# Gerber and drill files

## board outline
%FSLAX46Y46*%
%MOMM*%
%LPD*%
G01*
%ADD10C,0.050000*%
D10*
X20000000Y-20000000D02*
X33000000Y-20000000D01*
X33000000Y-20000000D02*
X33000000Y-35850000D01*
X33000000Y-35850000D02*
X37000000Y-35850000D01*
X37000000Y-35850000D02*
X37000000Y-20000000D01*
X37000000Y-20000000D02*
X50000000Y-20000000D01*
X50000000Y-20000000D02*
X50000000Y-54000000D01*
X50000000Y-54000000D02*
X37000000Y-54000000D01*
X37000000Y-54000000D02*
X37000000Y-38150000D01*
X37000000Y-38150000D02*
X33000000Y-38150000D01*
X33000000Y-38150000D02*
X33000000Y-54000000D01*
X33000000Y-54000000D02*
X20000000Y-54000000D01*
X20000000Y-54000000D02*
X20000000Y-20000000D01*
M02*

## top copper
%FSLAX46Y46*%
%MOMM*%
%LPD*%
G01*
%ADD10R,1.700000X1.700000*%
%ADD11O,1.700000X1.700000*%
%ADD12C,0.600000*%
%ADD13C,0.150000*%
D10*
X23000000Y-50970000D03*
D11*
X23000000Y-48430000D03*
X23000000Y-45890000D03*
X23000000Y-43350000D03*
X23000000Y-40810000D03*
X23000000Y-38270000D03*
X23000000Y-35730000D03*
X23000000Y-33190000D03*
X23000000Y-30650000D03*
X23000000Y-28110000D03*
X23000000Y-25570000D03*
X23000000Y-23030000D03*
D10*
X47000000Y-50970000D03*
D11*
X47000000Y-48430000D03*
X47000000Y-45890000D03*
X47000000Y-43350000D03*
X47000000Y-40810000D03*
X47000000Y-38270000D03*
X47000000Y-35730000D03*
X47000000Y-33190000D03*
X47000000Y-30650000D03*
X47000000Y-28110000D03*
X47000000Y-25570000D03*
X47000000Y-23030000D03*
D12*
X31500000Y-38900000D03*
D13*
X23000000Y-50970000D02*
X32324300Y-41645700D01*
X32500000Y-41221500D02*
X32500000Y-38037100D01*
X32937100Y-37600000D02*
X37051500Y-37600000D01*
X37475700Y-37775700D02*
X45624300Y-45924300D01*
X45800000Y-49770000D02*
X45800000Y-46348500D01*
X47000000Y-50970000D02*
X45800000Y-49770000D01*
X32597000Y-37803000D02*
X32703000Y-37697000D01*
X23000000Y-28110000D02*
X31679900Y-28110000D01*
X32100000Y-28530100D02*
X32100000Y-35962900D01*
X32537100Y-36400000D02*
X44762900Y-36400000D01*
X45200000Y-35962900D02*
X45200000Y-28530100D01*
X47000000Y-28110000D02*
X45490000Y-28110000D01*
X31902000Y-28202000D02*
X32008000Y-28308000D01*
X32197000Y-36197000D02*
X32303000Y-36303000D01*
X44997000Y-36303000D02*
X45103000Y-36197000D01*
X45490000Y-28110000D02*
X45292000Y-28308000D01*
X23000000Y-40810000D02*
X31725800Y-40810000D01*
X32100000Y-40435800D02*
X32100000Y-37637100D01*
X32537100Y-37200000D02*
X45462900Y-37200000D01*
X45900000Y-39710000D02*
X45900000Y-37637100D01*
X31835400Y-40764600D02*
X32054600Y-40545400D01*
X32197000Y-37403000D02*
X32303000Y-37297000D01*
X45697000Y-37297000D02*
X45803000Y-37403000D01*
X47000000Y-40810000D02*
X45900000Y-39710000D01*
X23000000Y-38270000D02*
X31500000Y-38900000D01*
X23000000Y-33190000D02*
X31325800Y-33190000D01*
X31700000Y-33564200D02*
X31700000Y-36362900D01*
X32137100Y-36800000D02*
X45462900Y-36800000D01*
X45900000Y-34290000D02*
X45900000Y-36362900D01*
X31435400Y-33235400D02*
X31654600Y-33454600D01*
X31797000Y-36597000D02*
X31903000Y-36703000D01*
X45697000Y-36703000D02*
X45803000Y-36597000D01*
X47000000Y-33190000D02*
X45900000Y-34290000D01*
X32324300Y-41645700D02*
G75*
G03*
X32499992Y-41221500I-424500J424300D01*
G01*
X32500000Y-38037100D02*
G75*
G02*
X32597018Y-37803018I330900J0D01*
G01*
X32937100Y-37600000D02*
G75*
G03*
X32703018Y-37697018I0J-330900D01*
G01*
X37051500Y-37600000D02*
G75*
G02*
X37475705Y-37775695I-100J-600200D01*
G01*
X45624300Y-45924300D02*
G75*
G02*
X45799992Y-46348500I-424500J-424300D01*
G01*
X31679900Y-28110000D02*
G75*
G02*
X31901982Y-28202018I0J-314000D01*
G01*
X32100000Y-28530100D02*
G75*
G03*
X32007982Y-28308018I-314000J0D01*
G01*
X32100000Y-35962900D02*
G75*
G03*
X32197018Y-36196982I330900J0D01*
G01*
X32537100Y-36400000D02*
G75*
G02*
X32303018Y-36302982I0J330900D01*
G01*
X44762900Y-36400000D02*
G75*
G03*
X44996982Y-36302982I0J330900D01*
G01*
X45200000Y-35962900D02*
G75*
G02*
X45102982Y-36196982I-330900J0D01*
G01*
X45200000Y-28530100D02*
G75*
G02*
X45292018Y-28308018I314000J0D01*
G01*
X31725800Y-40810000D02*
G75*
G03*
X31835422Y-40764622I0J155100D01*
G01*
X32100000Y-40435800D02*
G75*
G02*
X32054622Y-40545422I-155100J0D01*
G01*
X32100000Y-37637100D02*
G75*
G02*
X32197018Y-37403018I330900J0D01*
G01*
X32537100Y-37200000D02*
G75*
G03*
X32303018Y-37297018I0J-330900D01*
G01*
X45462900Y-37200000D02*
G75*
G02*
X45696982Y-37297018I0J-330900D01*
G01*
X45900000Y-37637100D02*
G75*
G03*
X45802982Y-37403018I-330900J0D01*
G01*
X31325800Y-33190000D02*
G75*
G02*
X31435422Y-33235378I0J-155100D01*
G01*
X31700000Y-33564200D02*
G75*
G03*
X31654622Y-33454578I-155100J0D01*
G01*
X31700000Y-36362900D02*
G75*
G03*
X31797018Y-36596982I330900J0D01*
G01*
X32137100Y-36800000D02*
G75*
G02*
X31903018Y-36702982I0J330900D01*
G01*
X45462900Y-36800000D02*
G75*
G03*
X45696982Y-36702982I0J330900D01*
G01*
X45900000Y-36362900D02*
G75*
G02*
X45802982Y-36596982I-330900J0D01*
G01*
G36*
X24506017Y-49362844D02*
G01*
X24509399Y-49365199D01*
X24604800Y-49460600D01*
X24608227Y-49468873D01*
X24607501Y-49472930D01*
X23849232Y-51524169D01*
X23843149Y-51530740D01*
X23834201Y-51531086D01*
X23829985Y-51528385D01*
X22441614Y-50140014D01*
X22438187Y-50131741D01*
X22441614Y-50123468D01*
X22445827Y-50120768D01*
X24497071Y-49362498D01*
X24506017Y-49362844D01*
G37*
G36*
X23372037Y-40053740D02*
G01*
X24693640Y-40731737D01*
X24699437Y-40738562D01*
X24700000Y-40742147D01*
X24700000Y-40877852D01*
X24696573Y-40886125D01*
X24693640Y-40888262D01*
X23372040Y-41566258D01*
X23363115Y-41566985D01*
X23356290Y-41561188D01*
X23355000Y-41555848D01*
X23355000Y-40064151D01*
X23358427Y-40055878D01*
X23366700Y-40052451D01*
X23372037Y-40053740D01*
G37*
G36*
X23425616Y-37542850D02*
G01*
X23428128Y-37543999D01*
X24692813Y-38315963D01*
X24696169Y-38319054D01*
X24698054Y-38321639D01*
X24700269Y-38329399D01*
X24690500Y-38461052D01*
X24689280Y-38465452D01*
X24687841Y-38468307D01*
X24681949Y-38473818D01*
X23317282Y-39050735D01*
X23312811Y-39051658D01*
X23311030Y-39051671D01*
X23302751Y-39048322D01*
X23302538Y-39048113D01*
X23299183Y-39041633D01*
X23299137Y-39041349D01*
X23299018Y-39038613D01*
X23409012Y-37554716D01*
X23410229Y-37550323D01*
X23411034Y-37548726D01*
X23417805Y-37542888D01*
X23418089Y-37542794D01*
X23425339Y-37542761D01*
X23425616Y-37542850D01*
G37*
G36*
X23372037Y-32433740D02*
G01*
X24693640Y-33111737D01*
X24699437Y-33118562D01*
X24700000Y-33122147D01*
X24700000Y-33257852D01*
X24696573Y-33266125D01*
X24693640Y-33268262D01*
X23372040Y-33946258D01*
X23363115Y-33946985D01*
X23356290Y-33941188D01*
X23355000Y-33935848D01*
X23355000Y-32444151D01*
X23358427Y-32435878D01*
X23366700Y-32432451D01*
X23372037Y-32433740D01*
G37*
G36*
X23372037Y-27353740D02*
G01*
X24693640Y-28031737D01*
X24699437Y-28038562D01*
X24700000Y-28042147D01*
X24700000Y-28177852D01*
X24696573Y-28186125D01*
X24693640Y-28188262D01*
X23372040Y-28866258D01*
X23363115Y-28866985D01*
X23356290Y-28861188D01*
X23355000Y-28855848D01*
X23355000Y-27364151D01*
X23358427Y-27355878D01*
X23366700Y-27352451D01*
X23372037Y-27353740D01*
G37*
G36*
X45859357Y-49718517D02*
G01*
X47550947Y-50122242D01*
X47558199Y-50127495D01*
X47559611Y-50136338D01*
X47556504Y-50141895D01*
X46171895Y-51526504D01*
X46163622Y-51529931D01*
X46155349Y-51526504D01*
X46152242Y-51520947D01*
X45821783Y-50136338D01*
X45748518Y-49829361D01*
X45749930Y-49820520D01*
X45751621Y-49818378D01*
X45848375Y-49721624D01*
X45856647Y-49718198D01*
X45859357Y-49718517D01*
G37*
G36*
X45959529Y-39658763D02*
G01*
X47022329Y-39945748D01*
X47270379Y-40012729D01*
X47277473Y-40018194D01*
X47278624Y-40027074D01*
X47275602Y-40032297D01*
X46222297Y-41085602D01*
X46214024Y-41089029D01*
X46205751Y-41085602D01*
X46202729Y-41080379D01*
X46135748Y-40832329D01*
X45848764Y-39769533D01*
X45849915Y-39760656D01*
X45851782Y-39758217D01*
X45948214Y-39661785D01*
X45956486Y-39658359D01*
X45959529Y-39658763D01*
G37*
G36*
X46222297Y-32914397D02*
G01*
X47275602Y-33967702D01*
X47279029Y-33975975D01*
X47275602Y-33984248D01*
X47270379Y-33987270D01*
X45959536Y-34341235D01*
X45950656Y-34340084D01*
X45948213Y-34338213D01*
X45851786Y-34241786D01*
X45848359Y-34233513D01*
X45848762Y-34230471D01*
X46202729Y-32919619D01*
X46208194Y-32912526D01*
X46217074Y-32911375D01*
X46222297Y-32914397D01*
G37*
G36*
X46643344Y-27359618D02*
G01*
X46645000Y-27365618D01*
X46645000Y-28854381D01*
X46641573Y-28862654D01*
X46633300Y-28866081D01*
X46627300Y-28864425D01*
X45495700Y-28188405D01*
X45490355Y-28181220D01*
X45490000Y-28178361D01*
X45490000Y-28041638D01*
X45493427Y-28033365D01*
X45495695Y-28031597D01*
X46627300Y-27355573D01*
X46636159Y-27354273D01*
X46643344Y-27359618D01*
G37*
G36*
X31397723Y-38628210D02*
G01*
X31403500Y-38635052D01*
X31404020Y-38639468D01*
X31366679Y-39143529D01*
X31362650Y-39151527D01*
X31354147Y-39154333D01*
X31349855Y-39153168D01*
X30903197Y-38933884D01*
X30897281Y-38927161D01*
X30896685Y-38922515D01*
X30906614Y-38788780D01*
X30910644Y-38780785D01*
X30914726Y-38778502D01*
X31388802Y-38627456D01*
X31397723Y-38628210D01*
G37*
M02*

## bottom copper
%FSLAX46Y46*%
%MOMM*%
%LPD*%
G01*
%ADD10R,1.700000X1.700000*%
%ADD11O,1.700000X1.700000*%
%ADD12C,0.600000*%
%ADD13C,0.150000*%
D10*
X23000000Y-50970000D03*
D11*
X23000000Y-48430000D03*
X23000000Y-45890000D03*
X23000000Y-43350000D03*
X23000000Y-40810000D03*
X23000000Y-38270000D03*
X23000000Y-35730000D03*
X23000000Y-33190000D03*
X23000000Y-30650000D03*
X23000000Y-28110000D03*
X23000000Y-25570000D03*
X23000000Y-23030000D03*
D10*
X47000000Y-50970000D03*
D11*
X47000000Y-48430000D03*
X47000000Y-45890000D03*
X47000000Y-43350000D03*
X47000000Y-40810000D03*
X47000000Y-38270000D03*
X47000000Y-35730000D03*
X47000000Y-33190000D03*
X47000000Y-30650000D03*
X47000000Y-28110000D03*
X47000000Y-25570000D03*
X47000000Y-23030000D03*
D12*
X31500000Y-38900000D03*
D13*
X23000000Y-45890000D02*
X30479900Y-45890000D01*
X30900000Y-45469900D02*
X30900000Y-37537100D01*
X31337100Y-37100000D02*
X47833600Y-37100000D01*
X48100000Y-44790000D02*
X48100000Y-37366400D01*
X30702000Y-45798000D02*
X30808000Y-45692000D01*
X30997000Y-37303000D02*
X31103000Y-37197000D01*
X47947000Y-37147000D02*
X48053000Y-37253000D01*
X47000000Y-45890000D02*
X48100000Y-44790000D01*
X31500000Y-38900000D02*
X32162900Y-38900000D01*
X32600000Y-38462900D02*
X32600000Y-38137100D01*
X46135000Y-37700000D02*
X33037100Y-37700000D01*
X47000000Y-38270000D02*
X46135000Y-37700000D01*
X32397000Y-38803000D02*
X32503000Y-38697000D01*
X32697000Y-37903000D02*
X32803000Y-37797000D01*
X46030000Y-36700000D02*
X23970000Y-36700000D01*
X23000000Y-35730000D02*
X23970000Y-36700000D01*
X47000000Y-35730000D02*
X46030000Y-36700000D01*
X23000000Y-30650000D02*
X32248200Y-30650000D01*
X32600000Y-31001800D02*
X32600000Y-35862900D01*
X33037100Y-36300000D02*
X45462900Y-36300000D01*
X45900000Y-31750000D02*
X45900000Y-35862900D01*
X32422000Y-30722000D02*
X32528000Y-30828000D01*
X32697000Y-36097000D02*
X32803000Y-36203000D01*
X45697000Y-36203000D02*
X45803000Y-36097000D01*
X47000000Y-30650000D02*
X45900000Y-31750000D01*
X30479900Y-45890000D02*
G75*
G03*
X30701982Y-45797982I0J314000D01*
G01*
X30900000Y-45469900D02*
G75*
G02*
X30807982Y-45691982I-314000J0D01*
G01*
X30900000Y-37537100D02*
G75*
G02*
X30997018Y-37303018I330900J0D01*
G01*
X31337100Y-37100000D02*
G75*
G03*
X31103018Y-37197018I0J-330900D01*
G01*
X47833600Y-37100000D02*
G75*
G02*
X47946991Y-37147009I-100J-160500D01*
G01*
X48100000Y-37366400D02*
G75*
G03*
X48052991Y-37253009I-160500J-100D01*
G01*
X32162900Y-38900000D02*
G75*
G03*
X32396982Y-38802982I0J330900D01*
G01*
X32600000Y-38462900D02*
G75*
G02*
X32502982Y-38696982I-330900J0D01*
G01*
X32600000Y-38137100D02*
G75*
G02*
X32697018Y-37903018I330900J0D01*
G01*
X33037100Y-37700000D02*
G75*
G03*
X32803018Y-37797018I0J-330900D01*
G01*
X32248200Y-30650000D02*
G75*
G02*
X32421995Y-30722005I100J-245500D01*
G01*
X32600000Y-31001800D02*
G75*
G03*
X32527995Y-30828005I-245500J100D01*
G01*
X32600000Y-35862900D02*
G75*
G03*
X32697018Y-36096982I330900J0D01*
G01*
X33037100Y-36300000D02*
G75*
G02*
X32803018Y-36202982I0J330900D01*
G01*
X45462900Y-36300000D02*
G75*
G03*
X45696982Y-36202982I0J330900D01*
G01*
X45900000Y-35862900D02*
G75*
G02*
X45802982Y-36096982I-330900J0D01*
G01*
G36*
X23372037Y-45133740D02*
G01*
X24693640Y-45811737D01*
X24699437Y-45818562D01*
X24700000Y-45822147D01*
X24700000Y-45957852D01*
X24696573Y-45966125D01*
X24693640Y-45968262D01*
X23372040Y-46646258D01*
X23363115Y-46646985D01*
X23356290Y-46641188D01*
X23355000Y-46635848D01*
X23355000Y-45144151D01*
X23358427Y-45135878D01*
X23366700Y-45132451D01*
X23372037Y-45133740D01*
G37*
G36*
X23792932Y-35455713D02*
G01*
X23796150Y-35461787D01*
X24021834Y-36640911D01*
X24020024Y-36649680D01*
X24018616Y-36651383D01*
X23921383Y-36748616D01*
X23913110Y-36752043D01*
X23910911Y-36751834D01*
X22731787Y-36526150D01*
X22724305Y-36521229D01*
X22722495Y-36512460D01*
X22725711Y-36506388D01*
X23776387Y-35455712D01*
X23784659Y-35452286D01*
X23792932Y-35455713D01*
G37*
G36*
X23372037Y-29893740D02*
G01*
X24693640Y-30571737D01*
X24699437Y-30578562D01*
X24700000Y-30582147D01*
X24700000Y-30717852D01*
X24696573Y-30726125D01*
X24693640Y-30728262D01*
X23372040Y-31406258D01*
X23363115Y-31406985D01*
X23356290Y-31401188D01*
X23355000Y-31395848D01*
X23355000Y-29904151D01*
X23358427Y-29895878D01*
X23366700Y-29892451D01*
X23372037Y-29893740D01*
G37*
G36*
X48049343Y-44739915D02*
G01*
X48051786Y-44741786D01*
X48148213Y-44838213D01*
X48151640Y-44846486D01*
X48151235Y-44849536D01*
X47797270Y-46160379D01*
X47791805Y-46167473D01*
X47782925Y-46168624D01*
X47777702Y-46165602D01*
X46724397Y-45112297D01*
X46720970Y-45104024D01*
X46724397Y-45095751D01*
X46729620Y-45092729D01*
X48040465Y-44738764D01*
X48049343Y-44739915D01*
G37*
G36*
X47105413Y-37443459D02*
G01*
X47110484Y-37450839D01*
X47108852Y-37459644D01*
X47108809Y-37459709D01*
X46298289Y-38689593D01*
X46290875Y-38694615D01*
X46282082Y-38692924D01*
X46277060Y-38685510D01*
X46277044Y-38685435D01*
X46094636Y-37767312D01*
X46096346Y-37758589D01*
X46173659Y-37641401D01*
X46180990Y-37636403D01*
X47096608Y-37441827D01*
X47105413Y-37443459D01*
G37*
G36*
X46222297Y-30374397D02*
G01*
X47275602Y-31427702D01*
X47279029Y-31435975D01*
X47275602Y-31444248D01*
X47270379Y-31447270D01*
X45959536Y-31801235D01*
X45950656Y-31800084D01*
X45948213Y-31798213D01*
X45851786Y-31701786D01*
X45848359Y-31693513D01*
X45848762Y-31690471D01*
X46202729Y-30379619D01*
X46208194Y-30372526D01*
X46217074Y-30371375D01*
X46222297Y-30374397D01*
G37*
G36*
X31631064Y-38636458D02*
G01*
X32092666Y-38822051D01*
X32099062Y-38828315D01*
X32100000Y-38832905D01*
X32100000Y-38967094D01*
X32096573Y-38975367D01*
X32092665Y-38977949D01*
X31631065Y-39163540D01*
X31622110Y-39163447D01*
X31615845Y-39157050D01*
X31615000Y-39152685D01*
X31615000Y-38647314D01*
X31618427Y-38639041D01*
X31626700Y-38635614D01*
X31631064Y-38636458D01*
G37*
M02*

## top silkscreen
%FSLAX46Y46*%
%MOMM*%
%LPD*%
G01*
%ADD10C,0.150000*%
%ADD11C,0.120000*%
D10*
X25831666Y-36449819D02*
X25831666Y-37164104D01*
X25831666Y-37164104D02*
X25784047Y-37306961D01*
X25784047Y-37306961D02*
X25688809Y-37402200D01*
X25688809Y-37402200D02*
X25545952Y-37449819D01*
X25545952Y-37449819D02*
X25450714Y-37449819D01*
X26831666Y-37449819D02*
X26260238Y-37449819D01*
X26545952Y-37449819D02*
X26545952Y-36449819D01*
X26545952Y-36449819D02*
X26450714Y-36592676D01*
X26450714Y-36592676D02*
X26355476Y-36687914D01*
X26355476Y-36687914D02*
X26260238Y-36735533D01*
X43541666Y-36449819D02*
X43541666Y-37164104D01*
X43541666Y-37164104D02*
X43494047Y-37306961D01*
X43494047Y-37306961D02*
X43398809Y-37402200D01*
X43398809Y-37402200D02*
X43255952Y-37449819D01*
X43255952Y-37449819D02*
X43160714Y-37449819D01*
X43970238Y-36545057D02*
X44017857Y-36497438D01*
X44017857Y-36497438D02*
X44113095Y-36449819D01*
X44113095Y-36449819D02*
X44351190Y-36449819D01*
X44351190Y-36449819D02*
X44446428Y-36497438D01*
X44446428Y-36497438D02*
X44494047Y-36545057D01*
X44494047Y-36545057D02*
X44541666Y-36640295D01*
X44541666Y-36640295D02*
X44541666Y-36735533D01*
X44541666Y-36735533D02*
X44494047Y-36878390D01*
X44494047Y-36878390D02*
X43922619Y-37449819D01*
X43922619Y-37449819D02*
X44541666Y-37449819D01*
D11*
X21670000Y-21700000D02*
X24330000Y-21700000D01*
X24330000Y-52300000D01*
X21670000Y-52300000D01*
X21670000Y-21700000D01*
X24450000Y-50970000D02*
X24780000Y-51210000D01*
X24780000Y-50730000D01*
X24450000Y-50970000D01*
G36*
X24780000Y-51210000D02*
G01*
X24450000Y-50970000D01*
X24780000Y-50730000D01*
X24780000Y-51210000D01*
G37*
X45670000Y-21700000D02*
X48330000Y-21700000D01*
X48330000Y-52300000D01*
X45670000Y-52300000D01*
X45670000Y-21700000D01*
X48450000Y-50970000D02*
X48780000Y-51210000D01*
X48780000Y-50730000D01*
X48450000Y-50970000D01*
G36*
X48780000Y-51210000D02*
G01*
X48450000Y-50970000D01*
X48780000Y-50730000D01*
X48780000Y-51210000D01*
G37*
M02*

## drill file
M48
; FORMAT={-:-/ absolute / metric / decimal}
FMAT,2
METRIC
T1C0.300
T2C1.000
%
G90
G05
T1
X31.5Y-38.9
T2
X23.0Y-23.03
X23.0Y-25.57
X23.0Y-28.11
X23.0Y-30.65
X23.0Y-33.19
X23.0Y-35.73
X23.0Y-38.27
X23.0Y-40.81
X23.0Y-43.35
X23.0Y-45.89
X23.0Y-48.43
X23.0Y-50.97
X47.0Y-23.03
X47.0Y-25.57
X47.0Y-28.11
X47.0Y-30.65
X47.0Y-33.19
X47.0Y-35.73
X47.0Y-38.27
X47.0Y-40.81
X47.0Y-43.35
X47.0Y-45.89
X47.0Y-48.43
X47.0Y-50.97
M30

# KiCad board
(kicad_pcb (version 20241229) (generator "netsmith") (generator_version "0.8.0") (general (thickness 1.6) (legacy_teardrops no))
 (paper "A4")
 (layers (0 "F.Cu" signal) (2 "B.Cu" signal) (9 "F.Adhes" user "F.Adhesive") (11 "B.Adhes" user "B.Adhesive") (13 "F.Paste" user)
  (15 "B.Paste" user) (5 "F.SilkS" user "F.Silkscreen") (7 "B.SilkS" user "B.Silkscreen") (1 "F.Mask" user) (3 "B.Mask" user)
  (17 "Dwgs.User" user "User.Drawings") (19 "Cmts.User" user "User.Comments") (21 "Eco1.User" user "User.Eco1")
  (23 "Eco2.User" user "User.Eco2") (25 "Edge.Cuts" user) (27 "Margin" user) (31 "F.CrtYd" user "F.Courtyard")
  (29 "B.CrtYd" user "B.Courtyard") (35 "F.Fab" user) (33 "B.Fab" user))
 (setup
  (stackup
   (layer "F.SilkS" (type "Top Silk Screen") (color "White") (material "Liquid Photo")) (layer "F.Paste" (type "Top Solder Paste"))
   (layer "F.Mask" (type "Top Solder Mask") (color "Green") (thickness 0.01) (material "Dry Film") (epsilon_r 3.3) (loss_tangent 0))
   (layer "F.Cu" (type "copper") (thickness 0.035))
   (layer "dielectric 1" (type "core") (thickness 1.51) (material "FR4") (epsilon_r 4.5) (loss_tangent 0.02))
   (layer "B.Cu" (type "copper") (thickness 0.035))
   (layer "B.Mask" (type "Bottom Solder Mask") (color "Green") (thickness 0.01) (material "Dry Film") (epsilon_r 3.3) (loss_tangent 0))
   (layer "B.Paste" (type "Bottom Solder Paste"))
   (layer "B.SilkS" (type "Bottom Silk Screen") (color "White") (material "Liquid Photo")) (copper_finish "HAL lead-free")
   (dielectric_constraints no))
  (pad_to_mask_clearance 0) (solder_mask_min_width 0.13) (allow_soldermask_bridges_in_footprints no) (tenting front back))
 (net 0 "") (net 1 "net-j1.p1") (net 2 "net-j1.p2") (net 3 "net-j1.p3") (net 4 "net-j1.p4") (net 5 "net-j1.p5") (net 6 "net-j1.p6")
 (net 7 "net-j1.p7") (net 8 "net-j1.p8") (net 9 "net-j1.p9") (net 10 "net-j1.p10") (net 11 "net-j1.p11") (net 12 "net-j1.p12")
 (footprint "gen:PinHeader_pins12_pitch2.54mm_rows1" (layer "F.Cu") (at 23 50.97 180)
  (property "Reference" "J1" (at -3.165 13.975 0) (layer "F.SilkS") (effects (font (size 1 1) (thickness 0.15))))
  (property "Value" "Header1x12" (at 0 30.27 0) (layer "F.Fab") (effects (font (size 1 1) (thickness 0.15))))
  (pad "1" thru_hole rect (at 0 0 180) (size 1.7 1.7) (drill 1) (layers "*.Cu" "*.Mask") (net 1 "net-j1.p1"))
  (pad "2" thru_hole oval (at 0 2.54 180) (size 1.7 1.7) (drill 1) (layers "*.Cu" "*.Mask") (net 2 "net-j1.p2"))
  (pad "3" thru_hole oval (at 0 5.08 180) (size 1.7 1.7) (drill 1) (layers "*.Cu" "*.Mask") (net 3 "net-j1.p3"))
  (pad "4" thru_hole oval (at 0 7.62 180) (size 1.7 1.7) (drill 1) (layers "*.Cu" "*.Mask") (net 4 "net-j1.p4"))
  (pad "5" thru_hole oval (at 0 10.16 180) (size 1.7 1.7) (drill 1) (layers "*.Cu" "*.Mask") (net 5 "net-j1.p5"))
  (pad "6" thru_hole oval (at 0 12.7 180) (size 1.7 1.7) (drill 1) (layers "*.Cu" "*.Mask") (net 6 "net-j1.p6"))
  (pad "7" thru_hole oval (at 0 15.24 180) (size 1.7 1.7) (drill 1) (layers "*.Cu" "*.Mask") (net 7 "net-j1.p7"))
  (pad "8" thru_hole oval (at 0 17.78 180) (size 1.7 1.7) (drill 1) (layers "*.Cu" "*.Mask") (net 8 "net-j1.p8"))
  (pad "9" thru_hole oval (at 0 20.32 180) (size 1.7 1.7) (drill 1) (layers "*.Cu" "*.Mask") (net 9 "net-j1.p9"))
  (pad "10" thru_hole oval (at 0 22.86 180) (size 1.7 1.7) (drill 1) (layers "*.Cu" "*.Mask") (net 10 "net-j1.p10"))
  (pad "11" thru_hole oval (at 0 25.4 180) (size 1.7 1.7) (drill 1) (layers "*.Cu" "*.Mask") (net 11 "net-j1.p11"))
  (pad "12" thru_hole oval (at 0 27.94 180) (size 1.7 1.7) (drill 1) (layers "*.Cu" "*.Mask") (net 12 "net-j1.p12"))
  (fp_rect (start -1.33 -1.33) (end 1.33 29.27) (stroke (width 0.12) (type solid)) (fill no) (layer "F.SilkS"))
  (fp_poly (pts (xy -1.45 0) (xy -1.78 -0.24) (xy -1.78 0.24)) (stroke (width 0.12) (type solid)) (fill solid) (layer "F.SilkS")))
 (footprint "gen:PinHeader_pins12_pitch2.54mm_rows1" (layer "F.Cu") (at 47 50.97 180)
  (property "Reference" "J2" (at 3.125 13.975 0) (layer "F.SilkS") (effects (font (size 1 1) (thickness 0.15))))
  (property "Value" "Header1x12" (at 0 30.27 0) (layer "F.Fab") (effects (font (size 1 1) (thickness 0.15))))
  (pad "1" thru_hole rect (at 0 0 180) (size 1.7 1.7) (drill 1) (layers "*.Cu" "*.Mask") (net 1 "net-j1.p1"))
  (pad "2" thru_hole oval (at 0 2.54 180) (size 1.7 1.7) (drill 1) (layers "*.Cu" "*.Mask") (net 2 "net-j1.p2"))
  (pad "3" thru_hole oval (at 0 5.08 180) (size 1.7 1.7) (drill 1) (layers "*.Cu" "*.Mask") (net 3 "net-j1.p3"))
  (pad "4" thru_hole oval (at 0 7.62 180) (size 1.7 1.7) (drill 1) (layers "*.Cu" "*.Mask") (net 4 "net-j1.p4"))
  (pad "5" thru_hole oval (at 0 10.16 180) (size 1.7 1.7) (drill 1) (layers "*.Cu" "*.Mask") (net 5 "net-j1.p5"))
  (pad "6" thru_hole oval (at 0 12.7 180) (size 1.7 1.7) (drill 1) (layers "*.Cu" "*.Mask") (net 6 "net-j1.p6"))
  (pad "7" thru_hole oval (at 0 15.24 180) (size 1.7 1.7) (drill 1) (layers "*.Cu" "*.Mask") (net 7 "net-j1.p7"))
  (pad "8" thru_hole oval (at 0 17.78 180) (size 1.7 1.7) (drill 1) (layers "*.Cu" "*.Mask") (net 8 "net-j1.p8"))
  (pad "9" thru_hole oval (at 0 20.32 180) (size 1.7 1.7) (drill 1) (layers "*.Cu" "*.Mask") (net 9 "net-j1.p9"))
  (pad "10" thru_hole oval (at 0 22.86 180) (size 1.7 1.7) (drill 1) (layers "*.Cu" "*.Mask") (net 10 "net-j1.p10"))
  (pad "11" thru_hole oval (at 0 25.4 180) (size 1.7 1.7) (drill 1) (layers "*.Cu" "*.Mask") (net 11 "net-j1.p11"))
  (pad "12" thru_hole oval (at 0 27.94 180) (size 1.7 1.7) (drill 1) (layers "*.Cu" "*.Mask") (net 12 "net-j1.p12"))
  (fp_rect (start -1.33 -1.33) (end 1.33 29.27) (stroke (width 0.12) (type solid)) (fill no) (layer "F.SilkS"))
  (fp_poly (pts (xy -1.45 0) (xy -1.78 -0.24) (xy -1.78 0.24)) (stroke (width 0.12) (type solid)) (fill solid) (layer "F.SilkS")))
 (segment (start 23 50.97) (end 32.3243 41.6457) (width 0.15) (layer "F.Cu") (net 1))
 (segment (start 32.5 41.2215) (end 32.5 38.0371) (width 0.15) (layer "F.Cu") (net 1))
 (segment (start 32.9371 37.6) (end 37.0515 37.6) (width 0.15) (layer "F.Cu") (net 1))
 (segment (start 37.4757 37.7757) (end 45.6243 45.9243) (width 0.15) (layer "F.Cu") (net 1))
 (segment (start 45.8 49.77) (end 45.8 46.3485) (width 0.15) (layer "F.Cu") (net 1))
 (segment (start 47 50.97) (end 45.8 49.77) (width 0.15) (layer "F.Cu") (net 1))
 (segment (start 32.597 37.803) (end 32.703 37.697) (width 0.15) (layer "F.Cu") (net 1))
 (segment (start 23 28.11) (end 31.6799 28.11) (width 0.15) (layer "F.Cu") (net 10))
 (segment (start 32.1 28.5301) (end 32.1 35.9629) (width 0.15) (layer "F.Cu") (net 10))
 (segment (start 32.5371 36.4) (end 44.7629 36.4) (width 0.15) (layer "F.Cu") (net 10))
 (segment (start 45.2 35.9629) (end 45.2 28.5301) (width 0.15) (layer "F.Cu") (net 10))
 (segment (start 47 28.11) (end 45.49 28.11) (width 0.15) (layer "F.Cu") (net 10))
 (segment (start 31.902 28.202) (end 32.008 28.308) (width 0.15) (layer "F.Cu") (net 10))
 (segment (start 32.197 36.197) (end 32.303 36.303) (width 0.15) (layer "F.Cu") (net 10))
 (segment (start 44.997 36.303) (end 45.103 36.197) (width 0.15) (layer "F.Cu") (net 10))
 (segment (start 45.49 28.11) (end 45.292 28.308) (width 0.15) (layer "F.Cu") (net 10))
 (segment (start 23 45.89) (end 30.4799 45.89) (width 0.15) (layer "B.Cu") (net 3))
 (segment (start 30.9 45.4699) (end 30.9 37.5371) (width 0.15) (layer "B.Cu") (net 3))
 (segment (start 31.3371 37.1) (end 47.8336 37.1) (width 0.15) (layer "B.Cu") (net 3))
 (segment (start 48.1 44.79) (end 48.1 37.3664) (width 0.15) (layer "B.Cu") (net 3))
 (segment (start 30.702 45.798) (end 30.808 45.692) (width 0.15) (layer "B.Cu") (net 3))
 (segment (start 30.997 37.303) (end 31.103 37.197) (width 0.15) (layer "B.Cu") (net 3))
 (segment (start 47.947 37.147) (end 48.053 37.253) (width 0.15) (layer "B.Cu") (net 3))
 (segment (start 47 45.89) (end 48.1 44.79) (width 0.15) (layer "B.Cu") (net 3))
 (segment (start 23 40.81) (end 31.7258 40.81) (width 0.15) (layer "F.Cu") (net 5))
 (segment (start 32.1 40.4358) (end 32.1 37.6371) (width 0.15) (layer "F.Cu") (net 5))
 (segment (start 32.5371 37.2) (end 45.4629 37.2) (width 0.15) (layer "F.Cu") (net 5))
 (segment (start 45.9 39.71) (end 45.9 37.6371) (width 0.15) (layer "F.Cu") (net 5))
 (segment (start 31.8354 40.7646) (end 32.0546 40.5454) (width 0.15) (layer "F.Cu") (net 5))
 (segment (start 32.197 37.403) (end 32.303 37.297) (width 0.15) (layer "F.Cu") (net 5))
 (segment (start 45.697 37.297) (end 45.803 37.403) (width 0.15) (layer "F.Cu") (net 5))
 (segment (start 47 40.81) (end 45.9 39.71) (width 0.15) (layer "F.Cu") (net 5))
 (segment (start 23 38.27) (end 31.5 38.9) (width 0.15) (layer "F.Cu") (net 6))
 (segment (start 31.5 38.9) (end 32.1629 38.9) (width 0.15) (layer "B.Cu") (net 6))
 (segment (start 32.6 38.4629) (end 32.6 38.1371) (width 0.15) (layer "B.Cu") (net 6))
 (segment (start 46.135 37.7) (end 33.0371 37.7) (width 0.15) (layer "B.Cu") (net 6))
 (segment (start 47 38.27) (end 46.135 37.7) (width 0.15) (layer "B.Cu") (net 6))
 (segment (start 32.397 38.803) (end 32.503 38.697) (width 0.15) (layer "B.Cu") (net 6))
 (segment (start 32.697 37.903) (end 32.803 37.797) (width 0.15) (layer "B.Cu") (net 6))
 (segment (start 46.03 36.7) (end 23.97 36.7) (width 0.15) (layer "B.Cu") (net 7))
 (segment (start 23 35.73) (end 23.97 36.7) (width 0.15) (layer "B.Cu") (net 7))
 (segment (start 47 35.73) (end 46.03 36.7) (width 0.15) (layer "B.Cu") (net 7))
 (segment (start 23 33.19) (end 31.3258 33.19) (width 0.15) (layer "F.Cu") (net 8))
 (segment (start 31.7 33.5642) (end 31.7 36.3629) (width 0.15) (layer "F.Cu") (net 8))
 (segment (start 32.1371 36.8) (end 45.4629 36.8) (width 0.15) (layer "F.Cu") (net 8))
 (segment (start 45.9 34.29) (end 45.9 36.3629) (width 0.15) (layer "F.Cu") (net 8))
 (segment (start 31.4354 33.2354) (end 31.6546 33.4546) (width 0.15) (layer "F.Cu") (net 8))
 (segment (start 31.797 36.597) (end 31.903 36.703) (width 0.15) (layer "F.Cu") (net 8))
 (segment (start 45.697 36.703) (end 45.803 36.597) (width 0.15) (layer "F.Cu") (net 8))
 (segment (start 47 33.19) (end 45.9 34.29) (width 0.15) (layer "F.Cu") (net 8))
 (segment (start 23 30.65) (end 32.2482 30.65) (width 0.15) (layer "B.Cu") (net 9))
 (segment (start 32.6 31.0018) (end 32.6 35.8629) (width 0.15) (layer "B.Cu") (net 9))
 (segment (start 33.0371 36.3) (end 45.4629 36.3) (width 0.15) (layer "B.Cu") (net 9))
 (segment (start 45.9 31.75) (end 45.9 35.8629) (width 0.15) (layer "B.Cu") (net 9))
 (segment (start 32.422 30.722) (end 32.528 30.828) (width 0.15) (layer "B.Cu") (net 9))
 (segment (start 32.697 36.097) (end 32.803 36.203) (width 0.15) (layer "B.Cu") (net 9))
 (segment (start 45.697 36.203) (end 45.803 36.097) (width 0.15) (layer "B.Cu") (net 9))
 (segment (start 47 30.65) (end 45.9 31.75) (width 0.15) (layer "B.Cu") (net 9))
 (arc (start 32.3243 41.6457) (mid 32.4543 41.4511) (end 32.5 41.2215) (width 0.15) (layer "F.Cu") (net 1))
 (arc (start 32.5 38.0371) (mid 32.5252 37.9104) (end 32.597 37.803) (width 0.15) (layer "F.Cu") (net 1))
 (arc (start 32.9371 37.6) (mid 32.8104 37.6252) (end 32.703 37.697) (width 0.15) (layer "F.Cu") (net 1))
 (arc (start 37.0515 37.6) (mid 37.2811 37.6457) (end 37.4757 37.7757) (width 0.15) (layer "F.Cu") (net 1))
 (arc (start 45.6243 45.9243) (mid 45.7543 46.1189) (end 45.8 46.3485) (width 0.15) (layer "F.Cu") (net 1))
 (arc (start 31.6799 28.11) (mid 31.8001 28.1339) (end 31.902 28.202) (width 0.15) (layer "F.Cu") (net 10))
 (arc (start 32.1 28.5301) (mid 32.0761 28.4099) (end 32.008 28.308) (width 0.15) (layer "F.Cu") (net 10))
 (arc (start 32.1 35.9629) (mid 32.1252 36.0896) (end 32.197 36.197) (width 0.15) (layer "F.Cu") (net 10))
 (arc (start 32.5371 36.4) (mid 32.4104 36.3748) (end 32.303 36.303) (width 0.15) (layer "F.Cu") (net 10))
 (arc (start 44.7629 36.4) (mid 44.8896 36.3748) (end 44.997 36.303) (width 0.15) (layer "F.Cu") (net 10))
 (arc (start 45.2 35.9629) (mid 45.1748 36.0896) (end 45.103 36.197) (width 0.15) (layer "F.Cu") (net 10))
 (arc (start 45.2 28.5301) (mid 45.2239 28.4099) (end 45.292 28.308) (width 0.15) (layer "F.Cu") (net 10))
 (arc (start 30.4799 45.89) (mid 30.6001 45.8661) (end 30.702 45.798) (width 0.15) (layer "B.Cu") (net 3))
 (arc (start 30.9 45.4699) (mid 30.8761 45.5901) (end 30.808 45.692) (width 0.15) (layer "B.Cu") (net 3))
 (arc (start 30.9 37.5371) (mid 30.9252 37.4104) (end 30.997 37.303) (width 0.15) (layer "B.Cu") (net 3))
 (arc (start 31.3371 37.1) (mid 31.2104 37.1252) (end 31.103 37.197) (width 0.15) (layer "B.Cu") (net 3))
 (arc (start 47.8336 37.1) (mid 47.8949 37.1122) (end 47.947 37.147) (width 0.15) (layer "B.Cu") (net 3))
 (arc (start 48.1 37.3664) (mid 48.0878 37.3051) (end 48.053 37.253) (width 0.15) (layer "B.Cu") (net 3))
 (arc (start 31.7258 40.81) (mid 31.7851 40.7982) (end 31.8354 40.7646) (width 0.15) (layer "F.Cu") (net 5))
 (arc (start 32.1 40.4358) (mid 32.0882 40.4951) (end 32.0546 40.5454) (width 0.15) (layer "F.Cu") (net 5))
 (arc (start 32.1 37.6371) (mid 32.1252 37.5104) (end 32.197 37.403) (width 0.15) (layer "F.Cu") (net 5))
 (arc (start 32.5371 37.2) (mid 32.4104 37.2252) (end 32.303 37.297) (width 0.15) (layer "F.Cu") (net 5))
 (arc (start 45.4629 37.2) (mid 45.5896 37.2252) (end 45.697 37.297) (width 0.15) (layer "F.Cu") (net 5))
 (arc (start 45.9 37.6371) (mid 45.8748 37.5104) (end 45.803 37.403) (width 0.15) (layer "F.Cu") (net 5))
 (arc (start 32.1629 38.9) (mid 32.2896 38.8748) (end 32.397 38.803) (width 0.15) (layer "B.Cu") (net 6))
 (arc (start 32.6 38.4629) (mid 32.5748 38.5896) (end 32.503 38.697) (width 0.15) (layer "B.Cu") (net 6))
 (arc (start 32.6 38.1371) (mid 32.6252 38.0104) (end 32.697 37.903) (width 0.15) (layer "B.Cu") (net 6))
 (arc (start 33.0371 37.7) (mid 32.9104 37.7252) (end 32.803 37.797) (width 0.15) (layer "B.Cu") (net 6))
 (arc (start 31.3258 33.19) (mid 31.3851 33.2018) (end 31.4354 33.2354) (width 0.15) (layer "F.Cu") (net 8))
 (arc (start 31.7 33.5642) (mid 31.6882 33.5049) (end 31.6546 33.4546) (width 0.15) (layer "F.Cu") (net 8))
 (arc (start 31.7 36.3629) (mid 31.7252 36.4896) (end 31.797 36.597) (width 0.15) (layer "F.Cu") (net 8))
 (arc (start 32.1371 36.8) (mid 32.0104 36.7748) (end 31.903 36.703) (width 0.15) (layer "F.Cu") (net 8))
 (arc (start 45.4629 36.8) (mid 45.5896 36.7748) (end 45.697 36.703) (width 0.15) (layer "F.Cu") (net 8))
 (arc (start 45.9 36.3629) (mid 45.8748 36.4896) (end 45.803 36.597) (width 0.15) (layer "F.Cu") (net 8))
 (arc (start 32.2482 30.65) (mid 32.3423 30.6687) (end 32.422 30.722) (width 0.15) (layer "B.Cu") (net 9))
 (arc (start 32.6 31.0018) (mid 32.5813 30.9077) (end 32.528 30.828) (width 0.15) (layer "B.Cu") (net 9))
 (arc (start 32.6 35.8629) (mid 32.6252 35.9896) (end 32.697 36.097) (width 0.15) (layer "B.Cu") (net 9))
 (arc (start 33.0371 36.3) (mid 32.9104 36.2748) (end 32.803 36.203) (width 0.15) (layer "B.Cu") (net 9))
 (arc (start 45.4629 36.3) (mid 45.5896 36.2748) (end 45.697 36.203) (width 0.15) (layer "B.Cu") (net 9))
 (arc (start 45.9 35.8629) (mid 45.8748 35.9896) (end 45.803 36.097) (width 0.15) (layer "B.Cu") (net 9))
 (via (at 31.5 38.9) (size 0.6) (drill 0.3) (layers "F.Cu" "B.Cu") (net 6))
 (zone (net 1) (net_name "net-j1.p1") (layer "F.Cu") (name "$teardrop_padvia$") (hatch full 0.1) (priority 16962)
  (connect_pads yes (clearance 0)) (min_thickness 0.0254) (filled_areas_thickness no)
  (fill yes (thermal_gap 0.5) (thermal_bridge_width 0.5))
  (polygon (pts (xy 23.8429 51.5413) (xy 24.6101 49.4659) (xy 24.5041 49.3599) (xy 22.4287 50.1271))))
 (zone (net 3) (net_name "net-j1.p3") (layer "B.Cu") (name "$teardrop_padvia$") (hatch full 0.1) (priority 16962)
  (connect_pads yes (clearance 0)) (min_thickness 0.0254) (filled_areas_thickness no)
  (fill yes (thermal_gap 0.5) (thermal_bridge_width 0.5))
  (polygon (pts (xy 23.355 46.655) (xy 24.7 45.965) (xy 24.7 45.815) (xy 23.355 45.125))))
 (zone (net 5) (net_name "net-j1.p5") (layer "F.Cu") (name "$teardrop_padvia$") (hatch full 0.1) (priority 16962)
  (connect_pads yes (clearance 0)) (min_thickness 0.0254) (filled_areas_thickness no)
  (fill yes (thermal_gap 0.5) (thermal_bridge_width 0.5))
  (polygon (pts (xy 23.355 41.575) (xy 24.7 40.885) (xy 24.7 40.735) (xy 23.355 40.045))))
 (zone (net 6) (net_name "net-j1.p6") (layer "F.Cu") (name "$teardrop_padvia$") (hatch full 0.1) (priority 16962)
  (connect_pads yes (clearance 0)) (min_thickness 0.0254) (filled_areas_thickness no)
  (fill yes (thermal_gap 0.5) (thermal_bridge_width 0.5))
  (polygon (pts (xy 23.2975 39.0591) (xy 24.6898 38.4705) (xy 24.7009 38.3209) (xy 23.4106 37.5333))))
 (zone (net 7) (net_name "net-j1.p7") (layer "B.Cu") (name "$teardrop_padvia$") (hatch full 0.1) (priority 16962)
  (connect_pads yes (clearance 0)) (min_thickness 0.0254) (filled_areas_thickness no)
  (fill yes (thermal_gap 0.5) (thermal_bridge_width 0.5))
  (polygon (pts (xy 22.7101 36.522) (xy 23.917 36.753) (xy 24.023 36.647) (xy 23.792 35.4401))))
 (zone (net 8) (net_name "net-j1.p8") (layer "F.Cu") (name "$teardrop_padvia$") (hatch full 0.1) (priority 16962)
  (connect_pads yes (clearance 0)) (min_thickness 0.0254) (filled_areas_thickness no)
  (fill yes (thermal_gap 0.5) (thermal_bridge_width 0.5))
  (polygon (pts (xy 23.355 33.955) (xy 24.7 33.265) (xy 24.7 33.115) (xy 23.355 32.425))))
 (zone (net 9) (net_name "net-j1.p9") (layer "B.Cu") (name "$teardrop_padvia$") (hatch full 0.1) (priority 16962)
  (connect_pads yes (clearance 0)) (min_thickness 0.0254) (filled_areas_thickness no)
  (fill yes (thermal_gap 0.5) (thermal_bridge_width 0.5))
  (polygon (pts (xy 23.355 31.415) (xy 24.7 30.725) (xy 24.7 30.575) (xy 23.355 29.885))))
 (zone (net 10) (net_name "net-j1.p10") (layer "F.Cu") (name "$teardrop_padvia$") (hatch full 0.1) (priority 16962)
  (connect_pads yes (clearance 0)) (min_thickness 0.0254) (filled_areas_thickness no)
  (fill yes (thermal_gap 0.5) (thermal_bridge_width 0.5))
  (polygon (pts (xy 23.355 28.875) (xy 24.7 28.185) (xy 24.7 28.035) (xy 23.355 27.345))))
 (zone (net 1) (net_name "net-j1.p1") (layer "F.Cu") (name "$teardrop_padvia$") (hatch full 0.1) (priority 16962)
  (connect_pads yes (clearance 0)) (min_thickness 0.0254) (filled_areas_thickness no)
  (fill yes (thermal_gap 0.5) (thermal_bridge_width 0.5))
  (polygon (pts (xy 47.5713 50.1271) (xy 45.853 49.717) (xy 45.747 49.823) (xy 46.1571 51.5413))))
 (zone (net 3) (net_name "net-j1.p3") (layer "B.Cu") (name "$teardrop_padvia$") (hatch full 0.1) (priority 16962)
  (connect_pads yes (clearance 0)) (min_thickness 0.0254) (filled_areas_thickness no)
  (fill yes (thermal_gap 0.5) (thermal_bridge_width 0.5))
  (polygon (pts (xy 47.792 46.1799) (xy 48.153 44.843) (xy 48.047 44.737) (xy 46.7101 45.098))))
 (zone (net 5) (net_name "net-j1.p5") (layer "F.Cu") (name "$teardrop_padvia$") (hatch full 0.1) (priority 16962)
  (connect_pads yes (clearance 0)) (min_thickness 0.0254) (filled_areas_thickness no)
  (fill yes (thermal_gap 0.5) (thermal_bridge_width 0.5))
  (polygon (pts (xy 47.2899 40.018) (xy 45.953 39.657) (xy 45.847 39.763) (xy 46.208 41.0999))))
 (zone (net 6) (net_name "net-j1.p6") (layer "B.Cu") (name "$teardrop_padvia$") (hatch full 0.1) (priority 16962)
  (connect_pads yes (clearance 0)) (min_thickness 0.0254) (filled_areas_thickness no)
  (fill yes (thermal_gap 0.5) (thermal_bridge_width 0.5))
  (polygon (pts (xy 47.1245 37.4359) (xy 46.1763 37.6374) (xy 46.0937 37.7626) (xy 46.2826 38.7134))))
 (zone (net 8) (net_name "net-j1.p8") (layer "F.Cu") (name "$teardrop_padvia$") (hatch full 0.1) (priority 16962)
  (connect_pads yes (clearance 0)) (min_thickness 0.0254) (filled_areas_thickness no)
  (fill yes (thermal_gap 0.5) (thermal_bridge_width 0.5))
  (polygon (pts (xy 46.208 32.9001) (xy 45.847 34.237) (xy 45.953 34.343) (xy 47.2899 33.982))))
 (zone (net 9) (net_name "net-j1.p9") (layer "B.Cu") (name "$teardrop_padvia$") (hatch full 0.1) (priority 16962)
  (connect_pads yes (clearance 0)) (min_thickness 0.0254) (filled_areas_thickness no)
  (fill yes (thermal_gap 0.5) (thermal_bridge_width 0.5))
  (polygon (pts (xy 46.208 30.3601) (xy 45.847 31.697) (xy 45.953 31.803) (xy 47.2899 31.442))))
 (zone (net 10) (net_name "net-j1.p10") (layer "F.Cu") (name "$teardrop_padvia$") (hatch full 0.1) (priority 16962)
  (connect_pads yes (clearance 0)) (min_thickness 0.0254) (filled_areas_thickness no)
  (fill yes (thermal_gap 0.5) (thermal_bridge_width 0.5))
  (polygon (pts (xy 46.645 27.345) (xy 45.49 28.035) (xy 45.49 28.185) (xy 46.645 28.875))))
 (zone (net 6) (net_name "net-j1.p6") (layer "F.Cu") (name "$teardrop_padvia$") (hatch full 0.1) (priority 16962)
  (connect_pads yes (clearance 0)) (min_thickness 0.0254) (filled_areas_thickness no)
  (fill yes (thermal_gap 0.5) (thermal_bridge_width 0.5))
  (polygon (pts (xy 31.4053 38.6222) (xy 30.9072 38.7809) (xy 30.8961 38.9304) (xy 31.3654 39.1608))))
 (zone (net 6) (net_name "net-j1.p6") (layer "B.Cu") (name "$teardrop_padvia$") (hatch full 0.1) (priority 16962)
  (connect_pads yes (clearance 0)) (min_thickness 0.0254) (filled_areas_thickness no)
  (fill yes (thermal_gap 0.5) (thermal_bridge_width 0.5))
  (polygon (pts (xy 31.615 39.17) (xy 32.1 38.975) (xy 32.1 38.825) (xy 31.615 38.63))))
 (gr_line (start 20 20) (end 33 20) (stroke (width 0.05) (type default)) (layer "Edge.Cuts"))
 (gr_line (start 33 20) (end 33 35.85) (stroke (width 0.05) (type default)) (layer "Edge.Cuts"))
 (gr_line (start 33 35.85) (end 37 35.85) (stroke (width 0.05) (type default)) (layer "Edge.Cuts"))
 (gr_line (start 37 35.85) (end 37 20) (stroke (width 0.05) (type default)) (layer "Edge.Cuts"))
 (gr_line (start 37 20) (end 50 20) (stroke (width 0.05) (type default)) (layer "Edge.Cuts"))
 (gr_line (start 50 20) (end 50 54) (stroke (width 0.05) (type default)) (layer "Edge.Cuts"))
 (gr_line (start 50 54) (end 37 54) (stroke (width 0.05) (type default)) (layer "Edge.Cuts"))
 (gr_line (start 37 54) (end 37 38.15) (stroke (width 0.05) (type default)) (layer "Edge.Cuts"))
 (gr_line (start 37 38.15) (end 33 38.15) (stroke (width 0.05) (type default)) (layer "Edge.Cuts"))
 (gr_line (start 33 38.15) (end 33 54) (stroke (width 0.05) (type default)) (layer "Edge.Cuts"))
 (gr_line (start 33 54) (end 20 54) (stroke (width 0.05) (type default)) (layer "Edge.Cuts"))
 (gr_line (start 20 54) (end 20 20) (stroke (width 0.05) (type default)) (layer "Edge.Cuts")))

